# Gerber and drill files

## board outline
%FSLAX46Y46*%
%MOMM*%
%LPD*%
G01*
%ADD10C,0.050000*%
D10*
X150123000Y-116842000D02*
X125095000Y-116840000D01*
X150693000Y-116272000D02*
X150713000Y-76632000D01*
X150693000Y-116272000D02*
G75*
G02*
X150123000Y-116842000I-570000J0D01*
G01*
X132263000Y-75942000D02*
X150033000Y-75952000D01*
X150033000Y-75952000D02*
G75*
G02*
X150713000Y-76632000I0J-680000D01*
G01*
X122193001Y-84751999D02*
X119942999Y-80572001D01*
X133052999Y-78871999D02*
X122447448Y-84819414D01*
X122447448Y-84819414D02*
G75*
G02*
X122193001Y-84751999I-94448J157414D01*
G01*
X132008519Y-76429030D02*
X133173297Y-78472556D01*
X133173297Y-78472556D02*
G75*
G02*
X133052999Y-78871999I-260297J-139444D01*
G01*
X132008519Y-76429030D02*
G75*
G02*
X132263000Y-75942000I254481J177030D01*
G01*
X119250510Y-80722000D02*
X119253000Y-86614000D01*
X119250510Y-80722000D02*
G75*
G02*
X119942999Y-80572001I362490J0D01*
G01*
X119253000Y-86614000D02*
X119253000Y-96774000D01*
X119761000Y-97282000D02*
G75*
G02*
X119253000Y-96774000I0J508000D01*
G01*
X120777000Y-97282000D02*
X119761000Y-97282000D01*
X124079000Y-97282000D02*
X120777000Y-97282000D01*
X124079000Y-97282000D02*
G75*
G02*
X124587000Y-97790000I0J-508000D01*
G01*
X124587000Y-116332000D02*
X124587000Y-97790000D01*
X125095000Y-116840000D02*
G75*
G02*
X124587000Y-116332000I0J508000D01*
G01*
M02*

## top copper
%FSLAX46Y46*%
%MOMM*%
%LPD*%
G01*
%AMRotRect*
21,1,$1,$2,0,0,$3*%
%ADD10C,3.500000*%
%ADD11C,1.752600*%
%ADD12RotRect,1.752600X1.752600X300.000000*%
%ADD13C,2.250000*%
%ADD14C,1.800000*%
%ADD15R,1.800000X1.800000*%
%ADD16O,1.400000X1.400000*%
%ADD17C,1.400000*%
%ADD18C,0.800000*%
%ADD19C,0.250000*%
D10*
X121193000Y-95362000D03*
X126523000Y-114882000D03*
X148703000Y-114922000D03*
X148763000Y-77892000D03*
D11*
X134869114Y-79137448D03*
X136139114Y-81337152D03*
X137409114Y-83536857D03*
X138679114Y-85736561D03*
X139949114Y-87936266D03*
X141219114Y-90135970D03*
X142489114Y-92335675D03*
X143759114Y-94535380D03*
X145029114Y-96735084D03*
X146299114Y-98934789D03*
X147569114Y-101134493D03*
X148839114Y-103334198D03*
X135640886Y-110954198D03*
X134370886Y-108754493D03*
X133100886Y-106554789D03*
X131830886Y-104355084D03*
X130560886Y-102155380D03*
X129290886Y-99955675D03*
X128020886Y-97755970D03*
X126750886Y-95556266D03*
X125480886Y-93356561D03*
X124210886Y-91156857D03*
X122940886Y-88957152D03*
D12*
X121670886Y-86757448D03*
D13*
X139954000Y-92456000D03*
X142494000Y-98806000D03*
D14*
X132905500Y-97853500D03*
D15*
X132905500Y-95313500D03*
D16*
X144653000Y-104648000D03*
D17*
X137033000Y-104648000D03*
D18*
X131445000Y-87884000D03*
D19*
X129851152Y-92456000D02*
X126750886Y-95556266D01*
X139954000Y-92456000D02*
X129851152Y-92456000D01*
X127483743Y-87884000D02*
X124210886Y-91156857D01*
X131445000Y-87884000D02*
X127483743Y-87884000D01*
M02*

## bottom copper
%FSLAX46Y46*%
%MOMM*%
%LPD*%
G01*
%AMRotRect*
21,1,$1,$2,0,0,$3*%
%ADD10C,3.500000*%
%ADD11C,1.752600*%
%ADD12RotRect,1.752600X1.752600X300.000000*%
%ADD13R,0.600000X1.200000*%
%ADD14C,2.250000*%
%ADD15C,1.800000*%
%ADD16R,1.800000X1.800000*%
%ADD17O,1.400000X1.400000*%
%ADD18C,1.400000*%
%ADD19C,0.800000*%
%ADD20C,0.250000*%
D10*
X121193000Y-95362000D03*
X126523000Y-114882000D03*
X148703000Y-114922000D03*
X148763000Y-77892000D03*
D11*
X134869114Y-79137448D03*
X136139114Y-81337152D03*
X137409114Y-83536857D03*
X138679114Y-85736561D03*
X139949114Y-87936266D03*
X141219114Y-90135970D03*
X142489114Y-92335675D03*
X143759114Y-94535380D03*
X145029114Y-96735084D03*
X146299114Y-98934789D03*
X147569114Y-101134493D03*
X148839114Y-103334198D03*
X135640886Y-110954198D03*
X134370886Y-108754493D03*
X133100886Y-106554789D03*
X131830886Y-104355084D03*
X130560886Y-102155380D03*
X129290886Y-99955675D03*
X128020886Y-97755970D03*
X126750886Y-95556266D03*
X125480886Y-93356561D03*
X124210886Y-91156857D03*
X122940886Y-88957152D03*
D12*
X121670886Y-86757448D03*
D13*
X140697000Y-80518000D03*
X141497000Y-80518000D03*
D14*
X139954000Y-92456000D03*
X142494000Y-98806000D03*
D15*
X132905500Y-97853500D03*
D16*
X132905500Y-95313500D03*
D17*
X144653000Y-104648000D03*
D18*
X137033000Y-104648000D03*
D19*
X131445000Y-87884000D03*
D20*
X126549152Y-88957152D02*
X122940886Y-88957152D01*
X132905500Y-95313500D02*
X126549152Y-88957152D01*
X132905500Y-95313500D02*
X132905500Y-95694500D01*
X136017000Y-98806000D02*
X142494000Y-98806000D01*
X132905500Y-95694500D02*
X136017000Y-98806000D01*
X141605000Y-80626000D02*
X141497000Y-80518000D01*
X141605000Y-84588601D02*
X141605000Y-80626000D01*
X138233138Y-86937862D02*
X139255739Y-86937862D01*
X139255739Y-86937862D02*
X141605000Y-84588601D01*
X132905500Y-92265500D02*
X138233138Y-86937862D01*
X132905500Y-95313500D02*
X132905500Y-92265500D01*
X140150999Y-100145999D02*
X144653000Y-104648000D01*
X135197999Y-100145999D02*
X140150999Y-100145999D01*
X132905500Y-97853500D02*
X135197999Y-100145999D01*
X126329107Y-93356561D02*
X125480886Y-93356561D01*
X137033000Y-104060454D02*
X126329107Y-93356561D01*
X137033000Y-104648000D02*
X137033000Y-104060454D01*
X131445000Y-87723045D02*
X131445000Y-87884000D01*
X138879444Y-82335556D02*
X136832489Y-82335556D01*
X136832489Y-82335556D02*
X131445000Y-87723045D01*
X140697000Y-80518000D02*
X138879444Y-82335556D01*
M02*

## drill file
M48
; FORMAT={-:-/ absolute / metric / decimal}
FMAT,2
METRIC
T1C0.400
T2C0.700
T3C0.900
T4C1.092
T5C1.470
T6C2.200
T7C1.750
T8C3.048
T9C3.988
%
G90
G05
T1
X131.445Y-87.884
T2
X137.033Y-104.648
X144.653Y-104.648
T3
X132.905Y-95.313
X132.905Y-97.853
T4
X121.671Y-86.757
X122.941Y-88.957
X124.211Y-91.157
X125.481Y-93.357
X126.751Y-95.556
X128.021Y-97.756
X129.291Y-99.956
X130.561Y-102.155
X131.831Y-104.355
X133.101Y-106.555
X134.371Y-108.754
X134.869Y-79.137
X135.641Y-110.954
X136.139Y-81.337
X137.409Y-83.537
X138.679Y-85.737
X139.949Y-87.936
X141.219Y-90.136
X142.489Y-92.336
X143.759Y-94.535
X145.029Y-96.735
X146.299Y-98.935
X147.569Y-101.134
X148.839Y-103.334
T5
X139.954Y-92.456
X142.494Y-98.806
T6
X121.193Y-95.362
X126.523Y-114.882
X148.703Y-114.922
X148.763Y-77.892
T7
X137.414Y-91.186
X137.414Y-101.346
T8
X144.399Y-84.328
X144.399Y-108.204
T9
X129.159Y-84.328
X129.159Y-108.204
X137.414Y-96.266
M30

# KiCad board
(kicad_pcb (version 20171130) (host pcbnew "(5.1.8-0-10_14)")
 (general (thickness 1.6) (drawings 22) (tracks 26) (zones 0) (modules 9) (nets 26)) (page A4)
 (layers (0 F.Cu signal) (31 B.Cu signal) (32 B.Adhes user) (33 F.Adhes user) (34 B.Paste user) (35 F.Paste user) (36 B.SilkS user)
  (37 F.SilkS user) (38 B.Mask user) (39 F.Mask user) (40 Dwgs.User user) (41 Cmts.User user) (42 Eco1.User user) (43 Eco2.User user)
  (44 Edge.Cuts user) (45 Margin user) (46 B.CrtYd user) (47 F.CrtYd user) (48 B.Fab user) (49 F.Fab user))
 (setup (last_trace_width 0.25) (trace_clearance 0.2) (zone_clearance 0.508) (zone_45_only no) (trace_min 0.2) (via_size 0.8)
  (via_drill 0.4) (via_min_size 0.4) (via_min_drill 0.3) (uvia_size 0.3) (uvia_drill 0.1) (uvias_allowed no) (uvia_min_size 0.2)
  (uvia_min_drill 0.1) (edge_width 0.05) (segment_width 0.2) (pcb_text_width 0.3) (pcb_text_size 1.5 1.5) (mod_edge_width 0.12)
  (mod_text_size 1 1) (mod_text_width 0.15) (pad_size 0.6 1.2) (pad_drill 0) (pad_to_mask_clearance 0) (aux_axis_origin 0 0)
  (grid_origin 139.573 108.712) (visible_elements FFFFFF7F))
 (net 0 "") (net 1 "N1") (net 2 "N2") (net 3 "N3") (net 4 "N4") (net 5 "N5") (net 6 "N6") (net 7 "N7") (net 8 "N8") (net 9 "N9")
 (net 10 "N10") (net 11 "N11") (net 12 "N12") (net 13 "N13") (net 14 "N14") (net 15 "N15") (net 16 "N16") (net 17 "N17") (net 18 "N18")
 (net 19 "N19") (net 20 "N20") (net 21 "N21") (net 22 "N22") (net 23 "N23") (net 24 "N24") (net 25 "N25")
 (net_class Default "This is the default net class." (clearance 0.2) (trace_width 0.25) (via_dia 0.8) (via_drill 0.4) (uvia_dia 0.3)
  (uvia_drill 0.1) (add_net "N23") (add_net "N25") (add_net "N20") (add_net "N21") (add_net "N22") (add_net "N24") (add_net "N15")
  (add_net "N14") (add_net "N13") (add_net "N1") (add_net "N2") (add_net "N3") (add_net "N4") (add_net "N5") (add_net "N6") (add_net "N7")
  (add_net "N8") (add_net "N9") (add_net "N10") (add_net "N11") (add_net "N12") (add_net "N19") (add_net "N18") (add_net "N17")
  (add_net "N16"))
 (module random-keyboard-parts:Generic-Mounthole (layer F.Cu) (at 121.193 95.362)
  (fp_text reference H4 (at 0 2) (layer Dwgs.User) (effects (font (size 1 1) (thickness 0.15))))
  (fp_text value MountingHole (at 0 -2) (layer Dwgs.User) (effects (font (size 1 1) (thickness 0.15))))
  (pad 1 thru_hole circle (at 0 0) (size 3.5 3.5) (drill 2.2) (layers *.Cu *.Mask)))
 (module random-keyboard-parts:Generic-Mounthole (layer F.Cu) (at 126.523 114.882)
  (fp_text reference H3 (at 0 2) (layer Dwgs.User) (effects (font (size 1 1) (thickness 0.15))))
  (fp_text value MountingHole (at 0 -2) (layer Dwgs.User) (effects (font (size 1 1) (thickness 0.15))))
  (pad 1 thru_hole circle (at 0 0) (size 3.5 3.5) (drill 2.2) (layers *.Cu *.Mask)))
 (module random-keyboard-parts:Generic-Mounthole (layer F.Cu) (at 148.703 114.922)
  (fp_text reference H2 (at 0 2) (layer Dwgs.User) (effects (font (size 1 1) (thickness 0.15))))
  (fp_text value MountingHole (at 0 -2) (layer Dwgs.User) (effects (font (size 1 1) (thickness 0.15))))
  (pad 1 thru_hole circle (at 0 0) (size 3.5 3.5) (drill 2.2) (layers *.Cu *.Mask)))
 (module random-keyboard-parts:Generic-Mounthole (layer F.Cu) (at 148.763 77.892)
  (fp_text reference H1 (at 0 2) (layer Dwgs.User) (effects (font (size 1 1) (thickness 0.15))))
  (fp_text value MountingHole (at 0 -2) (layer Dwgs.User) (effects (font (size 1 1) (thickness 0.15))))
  (pad 1 thru_hole circle (at 0 0) (size 3.5 3.5) (drill 2.2) (layers *.Cu *.Mask)))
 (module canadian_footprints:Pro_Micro (layer F.Cu) (at 134.493 93.726 30)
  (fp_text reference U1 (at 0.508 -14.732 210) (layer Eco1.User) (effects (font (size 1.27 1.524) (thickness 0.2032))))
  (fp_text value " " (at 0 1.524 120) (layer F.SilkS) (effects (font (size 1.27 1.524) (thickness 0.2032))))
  (pad 13 thru_hole circle (at 7.62 -12.446 300) (size 1.7526 1.7526) (drill 1.0922) (layers *.Cu *.SilkS *.Mask) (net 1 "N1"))
  (pad 14 thru_hole circle (at 7.62 -9.906 300) (size 1.7526 1.7526) (drill 1.0922) (layers *.Cu *.SilkS *.Mask) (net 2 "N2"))
  (pad 15 thru_hole circle (at 7.62 -7.366 300) (size 1.7526 1.7526) (drill 1.0922) (layers *.Cu *.SilkS *.Mask) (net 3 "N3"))
  (pad 16 thru_hole circle (at 7.62 -4.826 300) (size 1.7526 1.7526) (drill 1.0922) (layers *.Cu *.SilkS *.Mask) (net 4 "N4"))
  (pad 17 thru_hole circle (at 7.62 -2.286 300) (size 1.7526 1.7526) (drill 1.0922) (layers *.Cu *.SilkS *.Mask) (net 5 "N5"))
  (pad 18 thru_hole circle (at 7.62 0.254 300) (size 1.7526 1.7526) (drill 1.0922) (layers *.Cu *.SilkS *.Mask) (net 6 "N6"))
  (pad 19 thru_hole circle (at 7.62 2.794 300) (size 1.7526 1.7526) (drill 1.0922) (layers *.Cu *.SilkS *.Mask) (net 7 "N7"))
  (pad 20 thru_hole circle (at 7.62 5.334 300) (size 1.7526 1.7526) (drill 1.0922) (layers *.Cu *.SilkS *.Mask) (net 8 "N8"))
  (pad 21 thru_hole circle (at 7.62 7.874 300) (size 1.7526 1.7526) (drill 1.0922) (layers *.Cu *.SilkS *.Mask) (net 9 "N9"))
  (pad 22 thru_hole circle (at 7.62 10.414 300) (size 1.7526 1.7526) (drill 1.0922) (layers *.Cu *.SilkS *.Mask) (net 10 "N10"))
  (pad 23 thru_hole circle (at 7.62 12.954 300) (size 1.7526 1.7526) (drill 1.0922) (layers *.Cu *.SilkS *.Mask) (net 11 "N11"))
  (pad 24 thru_hole circle (at 7.62 15.494 300) (size 1.7526 1.7526) (drill 1.0922) (layers *.Cu *.SilkS *.Mask) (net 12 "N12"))
  (pad 12 thru_hole circle (at -7.62 15.494 300) (size 1.7526 1.7526) (drill 1.0922) (layers *.Cu *.SilkS *.Mask) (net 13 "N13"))
  (pad 11 thru_hole circle (at -7.62 12.954 300) (size 1.7526 1.7526) (drill 1.0922) (layers *.Cu *.SilkS *.Mask) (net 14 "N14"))
  (pad 10 thru_hole circle (at -7.62 10.414 300) (size 1.7526 1.7526) (drill 1.0922) (layers *.Cu *.SilkS *.Mask) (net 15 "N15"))
  (pad 9 thru_hole circle (at -7.62 7.874 300) (size 1.7526 1.7526) (drill 1.0922) (layers *.Cu *.SilkS *.Mask) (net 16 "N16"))
  (pad 8 thru_hole circle (at -7.62 5.334 300) (size 1.7526 1.7526) (drill 1.0922) (layers *.Cu *.SilkS *.Mask) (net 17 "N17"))
  (pad 7 thru_hole circle (at -7.62 2.794 300) (size 1.7526 1.7526) (drill 1.0922) (layers *.Cu *.SilkS *.Mask) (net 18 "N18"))
  (pad 6 thru_hole circle (at -7.62 0.254 300) (size 1.7526 1.7526) (drill 1.0922) (layers *.Cu *.SilkS *.Mask) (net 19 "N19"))
  (pad 5 thru_hole circle (at -7.62 -2.286 300) (size 1.7526 1.7526) (drill 1.0922) (layers *.Cu *.SilkS *.Mask) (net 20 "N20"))
  (pad 4 thru_hole circle (at -7.62 -4.826 300) (size 1.7526 1.7526) (drill 1.0922) (layers *.Cu *.SilkS *.Mask) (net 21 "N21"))
  (pad 3 thru_hole circle (at -7.62 -7.366 300) (size 1.7526 1.7526) (drill 1.0922) (layers *.Cu *.SilkS *.Mask) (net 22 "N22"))
  (pad 2 thru_hole circle (at -7.62 -9.906 300) (size 1.7526 1.7526) (drill 1.0922) (layers *.Cu *.SilkS *.Mask) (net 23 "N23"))
  (pad 1 thru_hole rect (at -7.62 -12.446 300) (size 1.7526 1.7526) (drill 1.0922) (layers *.Cu *.SilkS *.Mask) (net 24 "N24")))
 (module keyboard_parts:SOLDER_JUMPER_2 (layer F.Cu) (at 141.097 80.518)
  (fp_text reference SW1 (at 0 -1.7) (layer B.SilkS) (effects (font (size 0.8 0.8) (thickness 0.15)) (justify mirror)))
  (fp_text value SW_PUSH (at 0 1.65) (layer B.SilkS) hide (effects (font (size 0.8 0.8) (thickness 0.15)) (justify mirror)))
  (pad 1 smd rect (at -0.4 0) (size 0.6 1.2) (layers B.Cu B.Mask) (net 22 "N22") (clearance 0.1))
  (pad 2 smd rect (at 0.4 0) (size 0.6 1.2) (layers B.Cu B.Mask) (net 23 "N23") (clearance 0.1)))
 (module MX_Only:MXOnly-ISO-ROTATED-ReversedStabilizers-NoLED (layer F.Cu) (at 137.414 96.266)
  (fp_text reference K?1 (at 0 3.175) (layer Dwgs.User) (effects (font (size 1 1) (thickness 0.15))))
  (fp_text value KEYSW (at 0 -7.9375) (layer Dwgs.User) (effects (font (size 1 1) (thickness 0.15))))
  (pad "" np_thru_hole circle (at -8.255 -11.938) (size 3.9878 3.9878) (drill 3.9878) (layers *.Cu *.Mask))
  (pad "" np_thru_hole circle (at -8.255 11.938) (size 3.9878 3.9878) (drill 3.9878) (layers *.Cu *.Mask))
  (pad "" np_thru_hole circle (at 6.985 -11.938) (size 3.048 3.048) (drill 3.048) (layers *.Cu *.Mask))
  (pad "" np_thru_hole circle (at 6.985 11.938) (size 3.048 3.048) (drill 3.048) (layers *.Cu *.Mask))
  (pad "" np_thru_hole circle (at 0 5.08 48.0996) (size 1.75 1.75) (drill 1.75) (layers *.Cu *.Mask))
  (pad "" np_thru_hole circle (at 0 -5.08 48.0996) (size 1.75 1.75) (drill 1.75) (layers *.Cu *.Mask))
  (pad 1 thru_hole circle (at 2.54 -3.81) (size 2.25 2.25) (drill 1.47) (layers *.Cu B.Mask) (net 20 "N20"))
  (pad "" np_thru_hole circle (at 0 0) (size 3.9878 3.9878) (drill 3.9878) (layers *.Cu *.Mask))
  (pad 2 thru_hole circle (at 5.08 2.54) (size 2.25 2.25) (drill 1.47) (layers *.Cu B.Mask) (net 23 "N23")))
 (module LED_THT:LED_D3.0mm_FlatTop (layer F.Cu) (at 132.9055 95.3135 270)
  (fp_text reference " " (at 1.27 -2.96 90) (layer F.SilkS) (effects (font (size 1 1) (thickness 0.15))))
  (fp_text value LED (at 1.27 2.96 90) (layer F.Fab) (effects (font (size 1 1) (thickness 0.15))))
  (pad 2 thru_hole circle (at 2.54 0 270) (size 1.8 1.8) (drill 0.9) (layers *.Cu *.Mask) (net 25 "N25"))
  (pad 1 thru_hole rect (at 0 0 270) (size 1.8 1.8) (drill 0.9) (layers *.Cu *.Mask) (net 23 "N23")))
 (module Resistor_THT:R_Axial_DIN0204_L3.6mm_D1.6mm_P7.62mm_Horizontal (layer F.Cu) (at 137.033 104.648)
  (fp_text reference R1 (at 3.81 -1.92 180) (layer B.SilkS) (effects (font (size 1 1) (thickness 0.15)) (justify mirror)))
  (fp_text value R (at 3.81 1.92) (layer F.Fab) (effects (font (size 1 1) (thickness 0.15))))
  (pad 2 thru_hole oval (at 7.62 0) (size 1.4 1.4) (drill 0.7) (layers *.Cu *.Mask) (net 25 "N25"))
  (pad 1 thru_hole circle (at 0 0) (size 1.4 1.4) (drill 0.7) (layers *.Cu *.Mask) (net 21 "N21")))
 (gr_line (start 150.123 116.842) (end 125.095 116.84) (layer Edge.Cuts) (width 0.05))
 (gr_line (start 150.693 116.272) (end 150.713 76.632) (layer Edge.Cuts) (width 0.05))
 (gr_arc (start 150.123 116.272) (end 150.123 116.842) (angle -90) (layer Edge.Cuts) (width 0.05))
 (gr_line (start 132.263 75.942) (end 150.033 75.952) (layer Edge.Cuts) (width 0.05))
 (gr_arc (start 150.033 76.632) (end 150.713 76.632) (angle -90) (layer Edge.Cuts) (width 0.05))
 (gr_line (start 122.193001 84.751999) (end 119.942999 80.572001) (layer Edge.Cuts) (width 0.05))
 (gr_line (start 133.052999 78.871999) (end 122.447448 84.819414) (layer Edge.Cuts) (width 0.05))
 (gr_arc (start 122.353 84.662) (end 122.193001 84.751999) (angle -91.60600299) (layer Edge.Cuts) (width 0.05))
 (gr_line (start 132.008519 76.42903) (end 133.173297 78.472556) (layer Edge.Cuts) (width 0.05))
 (gr_arc (start 132.913 78.612) (end 133.052999 78.871999) (angle -89.87783434) (layer Edge.Cuts) (width 0.05))
 (gr_arc (start 132.263 76.252) (end 132.263 75.942) (angle -124.8244892) (layer Edge.Cuts) (width 0.05))
 (gr_line (start 119.25051 80.722) (end 119.253 86.614) (layer Edge.Cuts) (width 0.05))
 (gr_arc (start 119.613 80.722) (end 119.942999 80.572001) (angle -155.5560452) (layer Edge.Cuts) (width 0.05))
 (gr_line (start 119.253 86.614) (end 119.253 96.774) (layer Edge.Cuts) (width 0.05))
 (gr_arc (start 119.761 96.774) (end 119.253 96.774) (angle -90) (layer Edge.Cuts) (width 0.05))
 (gr_line (start 120.777 97.282) (end 119.761 97.282) (layer Edge.Cuts) (width 0.05))
 (gr_line (start 124.079 97.282) (end 120.777 97.282) (layer Edge.Cuts) (width 0.05))
 (gr_arc (start 124.079 97.79) (end 124.587 97.79) (angle -90) (layer Edge.Cuts) (width 0.05))
 (gr_line (start 124.587 116.332) (end 124.587 97.79) (layer Edge.Cuts) (width 0.05))
 (gr_arc (start 125.095 116.332) (end 124.587 116.332) (angle -90) (layer Edge.Cuts) (width 0.05))
 (segment (start 129.851152 92.456) (end 126.750886 95.556266) (width 0.25) (layer F.Cu) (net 20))
 (segment (start 139.954 92.456) (end 129.851152 92.456) (width 0.25) (layer F.Cu) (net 20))
 (segment (start 126.549152 88.957152) (end 122.940886 88.957152) (width 0.25) (layer B.Cu) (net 23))
 (segment (start 132.9055 95.3135) (end 126.549152 88.957152) (width 0.25) (layer B.Cu) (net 23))
 (segment (start 132.9055 95.3135) (end 132.9055 95.6945) (width 0.25) (layer B.Cu) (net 23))
 (segment (start 136.017 98.806) (end 142.494 98.806) (width 0.25) (layer B.Cu) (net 23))
 (segment (start 132.9055 95.6945) (end 136.017 98.806) (width 0.25) (layer B.Cu) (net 23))
 (segment (start 141.605 80.626) (end 141.497 80.518) (width 0.25) (layer B.Cu) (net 23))
 (segment (start 141.605 84.588601) (end 141.605 80.626) (width 0.25) (layer B.Cu) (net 23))
 (segment (start 138.233138 86.937862) (end 139.255739 86.937862) (width 0.25) (layer B.Cu) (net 23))
 (segment (start 139.255739 86.937862) (end 141.605 84.588601) (width 0.25) (layer B.Cu) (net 23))
 (segment (start 132.9055 92.2655) (end 138.233138 86.937862) (width 0.25) (layer B.Cu) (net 23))
 (segment (start 132.9055 95.3135) (end 132.9055 92.2655) (width 0.25) (layer B.Cu) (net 23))
 (segment (start 140.150999 100.145999) (end 144.653 104.648) (width 0.25) (layer B.Cu) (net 25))
 (segment (start 135.197999 100.145999) (end 140.150999 100.145999) (width 0.25) (layer B.Cu) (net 25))
 (segment (start 132.9055 97.8535) (end 135.197999 100.145999) (width 0.25) (layer B.Cu) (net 25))
 (segment (start 126.329107 93.356561) (end 125.480886 93.356561) (width 0.25) (layer B.Cu) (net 21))
 (segment (start 137.033 104.060454) (end 126.329107 93.356561) (width 0.25) (layer B.Cu) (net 21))
 (segment (start 137.033 104.648) (end 137.033 104.060454) (width 0.25) (layer B.Cu) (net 21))
 (segment (start 131.445 87.723045) (end 131.445 87.884) (width 0.25) (layer B.Cu) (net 22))
 (segment (start 138.879444 82.335556) (end 136.832489 82.335556) (width 0.25) (layer B.Cu) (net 22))
 (via (at 131.445 87.884) (size 0.8) (drill 0.4) (layers F.Cu B.Cu) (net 22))
 (segment (start 136.832489 82.335556) (end 131.445 87.723045) (width 0.25) (layer B.Cu) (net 22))
 (segment (start 140.697 80.518) (end 138.879444 82.335556) (width 0.25) (layer B.Cu) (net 22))
 (segment (start 127.483743 87.884) (end 124.210886 91.156857) (width 0.25) (layer F.Cu) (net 22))
 (segment (start 131.445 87.884) (end 127.483743 87.884) (width 0.25) (layer F.Cu) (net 22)))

